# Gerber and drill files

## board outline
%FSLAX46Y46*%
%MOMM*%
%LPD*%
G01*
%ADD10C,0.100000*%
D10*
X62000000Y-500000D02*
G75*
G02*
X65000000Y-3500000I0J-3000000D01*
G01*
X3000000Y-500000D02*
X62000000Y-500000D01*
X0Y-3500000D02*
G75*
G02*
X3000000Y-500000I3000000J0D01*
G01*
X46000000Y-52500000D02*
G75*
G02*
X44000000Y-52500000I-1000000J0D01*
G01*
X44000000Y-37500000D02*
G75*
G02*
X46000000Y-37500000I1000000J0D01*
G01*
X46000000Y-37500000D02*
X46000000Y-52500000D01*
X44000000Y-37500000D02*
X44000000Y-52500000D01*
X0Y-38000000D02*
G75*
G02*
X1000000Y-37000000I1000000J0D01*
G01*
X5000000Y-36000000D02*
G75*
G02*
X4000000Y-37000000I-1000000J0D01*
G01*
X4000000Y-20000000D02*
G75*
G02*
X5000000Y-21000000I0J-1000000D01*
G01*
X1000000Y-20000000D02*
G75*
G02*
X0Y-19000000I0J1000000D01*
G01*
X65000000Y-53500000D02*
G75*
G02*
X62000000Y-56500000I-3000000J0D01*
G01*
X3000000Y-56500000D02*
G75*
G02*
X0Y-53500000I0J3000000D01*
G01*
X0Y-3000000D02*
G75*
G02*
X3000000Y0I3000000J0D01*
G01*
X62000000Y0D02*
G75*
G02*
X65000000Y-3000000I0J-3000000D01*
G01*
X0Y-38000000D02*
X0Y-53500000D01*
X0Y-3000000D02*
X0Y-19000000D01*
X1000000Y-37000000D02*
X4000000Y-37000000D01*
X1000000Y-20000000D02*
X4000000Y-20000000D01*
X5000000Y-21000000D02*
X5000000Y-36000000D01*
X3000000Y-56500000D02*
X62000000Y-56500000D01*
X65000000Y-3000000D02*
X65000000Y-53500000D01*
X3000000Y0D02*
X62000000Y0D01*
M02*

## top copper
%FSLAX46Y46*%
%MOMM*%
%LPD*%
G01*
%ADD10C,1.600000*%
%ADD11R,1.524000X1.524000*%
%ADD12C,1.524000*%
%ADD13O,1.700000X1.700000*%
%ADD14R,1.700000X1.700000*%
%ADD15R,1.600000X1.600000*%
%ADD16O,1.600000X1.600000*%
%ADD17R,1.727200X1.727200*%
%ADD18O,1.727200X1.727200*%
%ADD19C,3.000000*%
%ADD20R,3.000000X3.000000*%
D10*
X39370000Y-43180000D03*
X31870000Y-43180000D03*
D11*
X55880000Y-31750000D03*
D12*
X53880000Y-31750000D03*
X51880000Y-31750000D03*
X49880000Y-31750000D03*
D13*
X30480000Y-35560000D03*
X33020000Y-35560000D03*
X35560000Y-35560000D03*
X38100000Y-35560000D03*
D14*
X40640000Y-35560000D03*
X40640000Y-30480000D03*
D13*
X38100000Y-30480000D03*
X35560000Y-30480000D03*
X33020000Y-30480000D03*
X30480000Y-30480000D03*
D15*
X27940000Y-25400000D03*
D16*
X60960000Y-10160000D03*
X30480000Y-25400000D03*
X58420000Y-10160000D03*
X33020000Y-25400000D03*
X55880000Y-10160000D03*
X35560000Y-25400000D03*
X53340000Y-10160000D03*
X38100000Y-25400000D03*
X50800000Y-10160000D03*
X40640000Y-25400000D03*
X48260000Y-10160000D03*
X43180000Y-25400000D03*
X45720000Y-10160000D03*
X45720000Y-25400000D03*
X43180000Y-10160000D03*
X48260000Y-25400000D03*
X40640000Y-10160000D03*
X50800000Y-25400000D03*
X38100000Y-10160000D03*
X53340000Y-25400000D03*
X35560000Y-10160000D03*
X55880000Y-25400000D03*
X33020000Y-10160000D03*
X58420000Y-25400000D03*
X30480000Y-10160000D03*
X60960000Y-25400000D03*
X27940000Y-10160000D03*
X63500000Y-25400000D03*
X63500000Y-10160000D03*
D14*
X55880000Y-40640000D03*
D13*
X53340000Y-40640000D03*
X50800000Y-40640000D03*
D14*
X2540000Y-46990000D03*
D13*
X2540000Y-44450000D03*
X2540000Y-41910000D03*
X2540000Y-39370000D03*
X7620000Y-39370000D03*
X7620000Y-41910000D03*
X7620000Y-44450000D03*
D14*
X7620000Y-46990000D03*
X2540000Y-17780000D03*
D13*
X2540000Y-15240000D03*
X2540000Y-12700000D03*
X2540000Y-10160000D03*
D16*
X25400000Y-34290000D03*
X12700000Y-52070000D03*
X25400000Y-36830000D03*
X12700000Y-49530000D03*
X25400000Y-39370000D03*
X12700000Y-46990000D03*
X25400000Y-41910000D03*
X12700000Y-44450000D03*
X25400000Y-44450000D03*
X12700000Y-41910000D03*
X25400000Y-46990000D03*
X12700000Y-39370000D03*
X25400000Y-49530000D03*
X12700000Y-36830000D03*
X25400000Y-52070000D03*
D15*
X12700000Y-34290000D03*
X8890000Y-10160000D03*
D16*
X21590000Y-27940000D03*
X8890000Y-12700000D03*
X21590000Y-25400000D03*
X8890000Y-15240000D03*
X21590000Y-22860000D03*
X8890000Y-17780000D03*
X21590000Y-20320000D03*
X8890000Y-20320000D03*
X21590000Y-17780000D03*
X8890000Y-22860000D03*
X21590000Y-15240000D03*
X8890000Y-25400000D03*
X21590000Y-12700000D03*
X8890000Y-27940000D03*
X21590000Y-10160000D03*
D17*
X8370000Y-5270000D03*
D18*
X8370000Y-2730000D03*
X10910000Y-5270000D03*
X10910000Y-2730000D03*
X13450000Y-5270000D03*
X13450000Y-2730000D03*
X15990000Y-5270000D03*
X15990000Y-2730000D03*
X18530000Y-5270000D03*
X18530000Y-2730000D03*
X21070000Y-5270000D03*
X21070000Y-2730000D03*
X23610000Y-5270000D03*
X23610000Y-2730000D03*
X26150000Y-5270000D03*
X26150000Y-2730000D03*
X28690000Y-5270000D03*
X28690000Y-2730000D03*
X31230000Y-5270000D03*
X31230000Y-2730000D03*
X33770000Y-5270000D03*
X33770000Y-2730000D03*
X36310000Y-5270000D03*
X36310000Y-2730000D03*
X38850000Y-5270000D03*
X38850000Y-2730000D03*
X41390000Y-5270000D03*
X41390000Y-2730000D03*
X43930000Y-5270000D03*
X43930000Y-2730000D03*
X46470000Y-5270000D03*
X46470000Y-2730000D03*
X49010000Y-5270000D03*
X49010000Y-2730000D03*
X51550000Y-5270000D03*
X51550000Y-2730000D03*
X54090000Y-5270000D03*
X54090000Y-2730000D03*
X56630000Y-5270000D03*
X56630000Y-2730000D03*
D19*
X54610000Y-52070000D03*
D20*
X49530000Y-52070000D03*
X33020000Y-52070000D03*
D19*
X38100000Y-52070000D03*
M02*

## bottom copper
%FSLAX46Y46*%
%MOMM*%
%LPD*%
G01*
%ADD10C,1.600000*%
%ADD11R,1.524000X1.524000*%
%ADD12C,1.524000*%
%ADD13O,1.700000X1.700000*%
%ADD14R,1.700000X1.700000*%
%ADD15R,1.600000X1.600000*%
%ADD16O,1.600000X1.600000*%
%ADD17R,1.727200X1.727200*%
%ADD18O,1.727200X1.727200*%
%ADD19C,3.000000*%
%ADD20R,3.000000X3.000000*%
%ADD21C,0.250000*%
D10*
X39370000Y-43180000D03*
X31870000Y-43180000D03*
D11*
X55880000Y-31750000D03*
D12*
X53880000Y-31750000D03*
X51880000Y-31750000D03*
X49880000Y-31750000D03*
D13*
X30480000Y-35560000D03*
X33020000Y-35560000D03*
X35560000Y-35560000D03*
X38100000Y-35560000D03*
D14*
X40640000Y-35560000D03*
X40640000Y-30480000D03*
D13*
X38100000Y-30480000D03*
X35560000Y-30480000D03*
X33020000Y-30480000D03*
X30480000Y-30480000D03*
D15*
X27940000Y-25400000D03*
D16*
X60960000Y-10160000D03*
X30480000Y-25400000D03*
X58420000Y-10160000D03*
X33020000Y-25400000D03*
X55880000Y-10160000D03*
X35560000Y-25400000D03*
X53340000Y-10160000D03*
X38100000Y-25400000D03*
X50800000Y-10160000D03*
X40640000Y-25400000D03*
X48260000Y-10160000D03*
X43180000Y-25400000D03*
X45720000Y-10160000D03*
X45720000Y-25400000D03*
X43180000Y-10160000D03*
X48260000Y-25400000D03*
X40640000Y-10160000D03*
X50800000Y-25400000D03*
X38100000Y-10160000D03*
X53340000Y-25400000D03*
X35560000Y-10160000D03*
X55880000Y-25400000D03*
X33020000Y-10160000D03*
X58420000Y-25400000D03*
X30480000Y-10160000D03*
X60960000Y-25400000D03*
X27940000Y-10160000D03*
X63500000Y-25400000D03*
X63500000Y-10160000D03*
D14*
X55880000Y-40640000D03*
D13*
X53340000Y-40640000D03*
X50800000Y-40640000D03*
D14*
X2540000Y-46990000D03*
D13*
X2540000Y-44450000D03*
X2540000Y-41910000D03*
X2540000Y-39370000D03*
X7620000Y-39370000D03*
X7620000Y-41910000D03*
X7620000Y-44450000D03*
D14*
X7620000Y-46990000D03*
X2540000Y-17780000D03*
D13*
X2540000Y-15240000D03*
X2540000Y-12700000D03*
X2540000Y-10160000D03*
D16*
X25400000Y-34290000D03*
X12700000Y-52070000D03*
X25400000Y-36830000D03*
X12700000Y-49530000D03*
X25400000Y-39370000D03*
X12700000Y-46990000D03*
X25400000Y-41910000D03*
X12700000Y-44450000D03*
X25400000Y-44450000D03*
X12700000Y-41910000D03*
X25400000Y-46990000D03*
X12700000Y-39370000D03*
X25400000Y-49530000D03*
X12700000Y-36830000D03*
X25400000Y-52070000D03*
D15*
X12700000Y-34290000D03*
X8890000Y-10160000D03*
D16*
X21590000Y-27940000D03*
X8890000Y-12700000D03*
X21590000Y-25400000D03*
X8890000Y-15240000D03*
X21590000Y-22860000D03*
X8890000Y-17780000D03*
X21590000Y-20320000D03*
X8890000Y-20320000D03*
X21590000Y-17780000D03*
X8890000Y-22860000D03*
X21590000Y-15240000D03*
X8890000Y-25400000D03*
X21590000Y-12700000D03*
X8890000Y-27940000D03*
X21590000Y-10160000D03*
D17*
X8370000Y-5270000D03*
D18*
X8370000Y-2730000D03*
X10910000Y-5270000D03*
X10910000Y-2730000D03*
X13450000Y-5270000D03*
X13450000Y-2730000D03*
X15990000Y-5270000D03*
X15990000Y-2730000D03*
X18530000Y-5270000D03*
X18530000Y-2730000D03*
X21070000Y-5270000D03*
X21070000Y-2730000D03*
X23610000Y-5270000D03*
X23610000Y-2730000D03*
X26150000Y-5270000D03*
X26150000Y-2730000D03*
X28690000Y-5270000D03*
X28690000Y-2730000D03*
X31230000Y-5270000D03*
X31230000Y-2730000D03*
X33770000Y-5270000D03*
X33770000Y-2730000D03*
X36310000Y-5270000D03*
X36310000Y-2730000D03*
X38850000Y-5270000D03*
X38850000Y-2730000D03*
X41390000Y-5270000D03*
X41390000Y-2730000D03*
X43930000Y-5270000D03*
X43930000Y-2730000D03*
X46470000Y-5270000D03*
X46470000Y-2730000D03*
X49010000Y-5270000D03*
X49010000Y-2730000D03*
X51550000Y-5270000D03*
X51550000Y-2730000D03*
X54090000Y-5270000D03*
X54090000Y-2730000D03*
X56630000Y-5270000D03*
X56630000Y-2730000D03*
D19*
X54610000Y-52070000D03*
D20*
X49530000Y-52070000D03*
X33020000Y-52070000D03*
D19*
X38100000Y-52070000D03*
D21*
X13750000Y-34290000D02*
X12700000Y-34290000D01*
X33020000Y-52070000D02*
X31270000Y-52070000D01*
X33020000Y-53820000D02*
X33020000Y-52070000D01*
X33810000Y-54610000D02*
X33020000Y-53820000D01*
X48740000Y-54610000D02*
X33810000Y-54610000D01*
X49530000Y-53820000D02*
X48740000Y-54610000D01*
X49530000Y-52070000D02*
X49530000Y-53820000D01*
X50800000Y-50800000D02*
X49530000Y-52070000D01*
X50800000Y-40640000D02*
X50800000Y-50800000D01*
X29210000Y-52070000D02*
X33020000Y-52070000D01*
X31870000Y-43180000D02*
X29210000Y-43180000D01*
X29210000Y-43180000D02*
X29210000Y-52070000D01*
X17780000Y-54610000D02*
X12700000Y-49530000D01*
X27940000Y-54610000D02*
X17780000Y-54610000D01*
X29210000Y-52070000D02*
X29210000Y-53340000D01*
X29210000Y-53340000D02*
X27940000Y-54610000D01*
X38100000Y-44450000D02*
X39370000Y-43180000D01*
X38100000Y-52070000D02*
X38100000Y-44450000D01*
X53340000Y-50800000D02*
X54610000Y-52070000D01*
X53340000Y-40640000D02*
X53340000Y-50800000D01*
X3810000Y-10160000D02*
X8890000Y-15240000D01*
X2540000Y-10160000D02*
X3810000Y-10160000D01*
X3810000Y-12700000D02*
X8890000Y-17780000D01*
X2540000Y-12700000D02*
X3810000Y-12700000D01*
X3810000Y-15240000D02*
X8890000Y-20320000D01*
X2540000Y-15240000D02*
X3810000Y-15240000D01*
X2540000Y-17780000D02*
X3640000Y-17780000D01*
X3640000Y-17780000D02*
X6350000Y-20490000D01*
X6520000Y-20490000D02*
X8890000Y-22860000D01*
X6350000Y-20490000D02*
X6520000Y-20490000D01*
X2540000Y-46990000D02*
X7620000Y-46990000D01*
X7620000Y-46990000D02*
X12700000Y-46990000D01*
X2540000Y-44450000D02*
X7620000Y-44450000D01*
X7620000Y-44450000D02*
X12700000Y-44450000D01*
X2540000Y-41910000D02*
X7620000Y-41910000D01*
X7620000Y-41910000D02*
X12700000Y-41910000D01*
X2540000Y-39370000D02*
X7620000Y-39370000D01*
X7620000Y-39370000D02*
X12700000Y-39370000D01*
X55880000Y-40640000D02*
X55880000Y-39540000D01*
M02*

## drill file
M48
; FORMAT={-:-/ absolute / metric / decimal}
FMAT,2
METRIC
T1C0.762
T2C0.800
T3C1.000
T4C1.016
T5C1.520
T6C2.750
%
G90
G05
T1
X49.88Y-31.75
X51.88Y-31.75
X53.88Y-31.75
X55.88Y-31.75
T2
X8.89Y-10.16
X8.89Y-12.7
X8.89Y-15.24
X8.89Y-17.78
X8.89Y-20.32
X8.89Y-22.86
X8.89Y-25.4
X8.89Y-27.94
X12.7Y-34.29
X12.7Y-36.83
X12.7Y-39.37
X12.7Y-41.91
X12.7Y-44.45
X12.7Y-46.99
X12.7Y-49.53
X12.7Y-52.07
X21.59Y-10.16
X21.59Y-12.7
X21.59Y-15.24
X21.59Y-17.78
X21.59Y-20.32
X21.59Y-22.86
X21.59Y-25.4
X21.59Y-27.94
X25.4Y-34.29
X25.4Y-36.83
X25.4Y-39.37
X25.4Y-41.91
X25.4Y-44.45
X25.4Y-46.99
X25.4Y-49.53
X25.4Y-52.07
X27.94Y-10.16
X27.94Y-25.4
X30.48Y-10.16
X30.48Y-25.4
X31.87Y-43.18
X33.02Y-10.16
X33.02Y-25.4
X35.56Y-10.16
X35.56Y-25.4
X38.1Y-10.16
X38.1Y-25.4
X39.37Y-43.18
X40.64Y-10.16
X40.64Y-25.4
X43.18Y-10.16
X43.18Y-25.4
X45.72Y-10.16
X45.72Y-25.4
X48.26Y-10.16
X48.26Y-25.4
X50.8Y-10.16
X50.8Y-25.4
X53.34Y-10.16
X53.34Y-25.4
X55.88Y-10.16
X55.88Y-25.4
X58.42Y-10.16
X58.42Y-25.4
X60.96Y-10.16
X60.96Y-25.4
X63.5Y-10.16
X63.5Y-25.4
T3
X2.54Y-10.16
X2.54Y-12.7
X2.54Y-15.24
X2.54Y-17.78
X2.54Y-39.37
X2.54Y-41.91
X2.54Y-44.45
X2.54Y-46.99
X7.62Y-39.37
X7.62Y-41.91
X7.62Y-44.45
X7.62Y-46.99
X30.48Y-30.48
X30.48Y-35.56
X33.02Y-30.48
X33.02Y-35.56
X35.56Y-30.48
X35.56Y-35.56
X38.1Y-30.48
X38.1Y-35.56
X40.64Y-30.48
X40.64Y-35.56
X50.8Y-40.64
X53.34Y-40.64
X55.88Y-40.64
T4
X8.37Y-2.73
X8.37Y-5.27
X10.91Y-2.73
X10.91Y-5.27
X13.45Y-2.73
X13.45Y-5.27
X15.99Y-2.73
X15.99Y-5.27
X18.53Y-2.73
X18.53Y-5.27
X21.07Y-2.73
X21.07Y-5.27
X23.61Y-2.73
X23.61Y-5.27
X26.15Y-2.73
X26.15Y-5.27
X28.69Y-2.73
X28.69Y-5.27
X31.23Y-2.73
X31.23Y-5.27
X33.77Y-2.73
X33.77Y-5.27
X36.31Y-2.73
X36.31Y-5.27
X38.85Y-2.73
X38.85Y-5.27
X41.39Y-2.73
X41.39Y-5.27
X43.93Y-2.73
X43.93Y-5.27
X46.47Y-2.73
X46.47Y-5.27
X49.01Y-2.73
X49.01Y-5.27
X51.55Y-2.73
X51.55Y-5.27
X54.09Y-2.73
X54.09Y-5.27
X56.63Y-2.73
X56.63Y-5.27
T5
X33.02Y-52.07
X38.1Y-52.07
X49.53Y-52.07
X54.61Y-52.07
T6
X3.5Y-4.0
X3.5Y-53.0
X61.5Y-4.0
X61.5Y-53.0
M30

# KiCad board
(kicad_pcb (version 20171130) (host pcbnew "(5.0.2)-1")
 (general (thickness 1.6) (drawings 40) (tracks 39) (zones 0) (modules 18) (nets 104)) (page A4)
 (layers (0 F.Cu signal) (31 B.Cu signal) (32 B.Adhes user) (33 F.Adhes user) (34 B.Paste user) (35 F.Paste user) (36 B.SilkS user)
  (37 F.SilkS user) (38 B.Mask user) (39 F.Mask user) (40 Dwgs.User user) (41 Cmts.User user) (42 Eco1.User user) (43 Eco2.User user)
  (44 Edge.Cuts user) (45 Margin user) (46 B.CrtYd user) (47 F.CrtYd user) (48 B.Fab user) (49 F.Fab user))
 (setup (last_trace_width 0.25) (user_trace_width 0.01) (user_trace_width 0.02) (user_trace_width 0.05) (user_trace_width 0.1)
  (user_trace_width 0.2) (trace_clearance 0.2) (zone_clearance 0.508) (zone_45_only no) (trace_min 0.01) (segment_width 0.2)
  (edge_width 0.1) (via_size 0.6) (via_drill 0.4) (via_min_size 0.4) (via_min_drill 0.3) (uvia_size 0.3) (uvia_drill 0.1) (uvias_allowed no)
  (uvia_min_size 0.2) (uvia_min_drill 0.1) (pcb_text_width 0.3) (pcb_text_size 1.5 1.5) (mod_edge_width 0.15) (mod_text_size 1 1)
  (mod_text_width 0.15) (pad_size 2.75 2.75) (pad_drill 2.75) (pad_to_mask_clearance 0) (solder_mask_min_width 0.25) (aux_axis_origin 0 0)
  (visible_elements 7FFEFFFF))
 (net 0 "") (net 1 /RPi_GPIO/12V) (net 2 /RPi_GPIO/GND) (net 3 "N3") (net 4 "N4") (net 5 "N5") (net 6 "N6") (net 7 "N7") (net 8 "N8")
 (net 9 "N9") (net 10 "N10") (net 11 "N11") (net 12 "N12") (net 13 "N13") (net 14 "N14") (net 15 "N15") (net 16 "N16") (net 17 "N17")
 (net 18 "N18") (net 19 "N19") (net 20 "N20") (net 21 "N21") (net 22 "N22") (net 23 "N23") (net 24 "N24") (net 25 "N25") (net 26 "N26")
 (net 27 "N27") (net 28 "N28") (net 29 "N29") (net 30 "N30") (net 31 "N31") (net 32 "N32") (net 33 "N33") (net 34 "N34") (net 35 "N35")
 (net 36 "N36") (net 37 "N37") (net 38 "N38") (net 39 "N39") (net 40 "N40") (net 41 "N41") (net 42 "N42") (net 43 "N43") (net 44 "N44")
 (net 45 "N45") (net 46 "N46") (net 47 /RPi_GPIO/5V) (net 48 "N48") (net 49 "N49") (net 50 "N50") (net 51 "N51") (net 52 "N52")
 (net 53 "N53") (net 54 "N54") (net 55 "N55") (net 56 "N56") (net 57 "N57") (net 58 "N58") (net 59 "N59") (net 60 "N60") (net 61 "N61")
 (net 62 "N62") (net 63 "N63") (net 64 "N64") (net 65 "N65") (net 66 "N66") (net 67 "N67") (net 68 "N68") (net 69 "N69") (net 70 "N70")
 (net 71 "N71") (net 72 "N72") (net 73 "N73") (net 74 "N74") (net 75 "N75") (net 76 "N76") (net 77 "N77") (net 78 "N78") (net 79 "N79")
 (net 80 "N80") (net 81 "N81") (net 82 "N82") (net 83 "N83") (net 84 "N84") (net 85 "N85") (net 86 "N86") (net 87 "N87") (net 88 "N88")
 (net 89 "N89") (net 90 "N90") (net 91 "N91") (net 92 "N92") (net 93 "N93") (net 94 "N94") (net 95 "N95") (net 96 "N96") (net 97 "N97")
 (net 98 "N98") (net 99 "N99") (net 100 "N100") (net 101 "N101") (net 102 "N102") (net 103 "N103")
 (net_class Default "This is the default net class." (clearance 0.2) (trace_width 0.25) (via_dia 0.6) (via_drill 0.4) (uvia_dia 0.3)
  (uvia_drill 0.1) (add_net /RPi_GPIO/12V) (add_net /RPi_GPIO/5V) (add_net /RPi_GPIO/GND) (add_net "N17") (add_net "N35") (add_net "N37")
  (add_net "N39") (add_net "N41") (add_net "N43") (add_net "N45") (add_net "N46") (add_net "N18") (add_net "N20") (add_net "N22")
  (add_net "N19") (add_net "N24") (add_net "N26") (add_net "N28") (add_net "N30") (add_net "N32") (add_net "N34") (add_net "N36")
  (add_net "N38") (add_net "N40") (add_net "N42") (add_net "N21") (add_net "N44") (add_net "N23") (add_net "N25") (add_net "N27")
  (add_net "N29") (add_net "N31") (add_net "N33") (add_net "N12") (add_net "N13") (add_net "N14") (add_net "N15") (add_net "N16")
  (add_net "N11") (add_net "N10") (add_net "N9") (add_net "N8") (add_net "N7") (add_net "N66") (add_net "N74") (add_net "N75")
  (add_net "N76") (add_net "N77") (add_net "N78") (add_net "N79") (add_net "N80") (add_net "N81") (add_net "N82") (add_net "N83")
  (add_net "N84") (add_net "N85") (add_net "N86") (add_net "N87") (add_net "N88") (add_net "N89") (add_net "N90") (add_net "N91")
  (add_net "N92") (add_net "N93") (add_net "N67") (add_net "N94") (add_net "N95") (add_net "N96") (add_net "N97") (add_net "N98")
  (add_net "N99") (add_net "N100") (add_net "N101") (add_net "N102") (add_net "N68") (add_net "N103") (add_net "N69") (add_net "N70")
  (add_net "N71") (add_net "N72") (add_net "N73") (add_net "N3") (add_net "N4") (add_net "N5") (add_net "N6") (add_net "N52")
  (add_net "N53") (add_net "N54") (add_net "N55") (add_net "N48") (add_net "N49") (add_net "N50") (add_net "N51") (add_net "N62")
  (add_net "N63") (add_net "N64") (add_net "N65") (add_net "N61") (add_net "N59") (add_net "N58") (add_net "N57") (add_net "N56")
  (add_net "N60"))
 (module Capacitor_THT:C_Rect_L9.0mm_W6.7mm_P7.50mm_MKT (layer F.Cu) (at 39.37 43.18 180)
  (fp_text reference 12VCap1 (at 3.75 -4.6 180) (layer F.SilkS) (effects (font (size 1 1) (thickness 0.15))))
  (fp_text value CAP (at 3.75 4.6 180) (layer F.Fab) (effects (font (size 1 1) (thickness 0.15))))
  (pad 1 thru_hole circle (at 0 0 180) (size 1.6 1.6) (drill 0.8) (layers *.Cu *.Mask) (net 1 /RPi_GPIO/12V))
  (pad 2 thru_hole circle (at 7.5 0 180) (size 1.6 1.6) (drill 0.8) (layers *.Cu *.Mask) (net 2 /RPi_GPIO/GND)))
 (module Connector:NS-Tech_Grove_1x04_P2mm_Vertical (layer F.Cu) (at 55.88 31.75 270)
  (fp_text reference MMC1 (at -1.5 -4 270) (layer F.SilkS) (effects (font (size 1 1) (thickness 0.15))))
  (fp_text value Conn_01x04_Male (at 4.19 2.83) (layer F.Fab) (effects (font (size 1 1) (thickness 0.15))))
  (pad 1 thru_hole rect (at 0 0 270) (size 1.524 1.524) (drill 0.762) (layers *.Cu *.Mask) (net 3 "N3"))
  (pad 2 thru_hole circle (at 0 2 270) (size 1.524 1.524) (drill 0.762) (layers *.Cu *.Mask) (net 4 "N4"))
  (pad 3 thru_hole circle (at 0 4 270) (size 1.524 1.524) (drill 0.762) (layers *.Cu *.Mask) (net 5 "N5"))
  (pad 4 thru_hole circle (at 0 6 270) (size 1.524 1.524) (drill 0.762) (layers *.Cu *.Mask) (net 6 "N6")))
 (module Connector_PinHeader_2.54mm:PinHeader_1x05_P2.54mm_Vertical (layer F.Cu) (at 40.64 35.56 270)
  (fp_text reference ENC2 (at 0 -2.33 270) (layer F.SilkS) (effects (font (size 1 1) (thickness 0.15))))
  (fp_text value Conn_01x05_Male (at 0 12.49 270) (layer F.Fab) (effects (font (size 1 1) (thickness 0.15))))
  (pad 5 thru_hole oval (at 0 10.16 270) (size 1.7 1.7) (drill 1) (layers *.Cu *.Mask) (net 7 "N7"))
  (pad 4 thru_hole oval (at 0 7.62 270) (size 1.7 1.7) (drill 1) (layers *.Cu *.Mask) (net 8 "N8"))
  (pad 3 thru_hole oval (at 0 5.08 270) (size 1.7 1.7) (drill 1) (layers *.Cu *.Mask) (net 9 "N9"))
  (pad 2 thru_hole oval (at 0 2.54 270) (size 1.7 1.7) (drill 1) (layers *.Cu *.Mask) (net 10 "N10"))
  (pad 1 thru_hole rect (at 0 0 270) (size 1.7 1.7) (drill 1) (layers *.Cu *.Mask) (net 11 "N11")))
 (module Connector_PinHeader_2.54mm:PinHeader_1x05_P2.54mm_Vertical (layer F.Cu) (at 40.64 30.48 270)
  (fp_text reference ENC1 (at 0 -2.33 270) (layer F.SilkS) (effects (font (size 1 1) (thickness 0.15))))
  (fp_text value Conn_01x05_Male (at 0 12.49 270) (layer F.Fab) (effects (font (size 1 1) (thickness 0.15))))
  (pad 1 thru_hole rect (at 0 0 270) (size 1.7 1.7) (drill 1) (layers *.Cu *.Mask) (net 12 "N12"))
  (pad 2 thru_hole oval (at 0 2.54 270) (size 1.7 1.7) (drill 1) (layers *.Cu *.Mask) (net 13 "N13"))
  (pad 3 thru_hole oval (at 0 5.08 270) (size 1.7 1.7) (drill 1) (layers *.Cu *.Mask) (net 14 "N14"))
  (pad 4 thru_hole oval (at 0 7.62 270) (size 1.7 1.7) (drill 1) (layers *.Cu *.Mask) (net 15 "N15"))
  (pad 5 thru_hole oval (at 0 10.16 270) (size 1.7 1.7) (drill 1) (layers *.Cu *.Mask) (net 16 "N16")))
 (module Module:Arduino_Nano (layer F.Cu) (at 27.94 25.4 90)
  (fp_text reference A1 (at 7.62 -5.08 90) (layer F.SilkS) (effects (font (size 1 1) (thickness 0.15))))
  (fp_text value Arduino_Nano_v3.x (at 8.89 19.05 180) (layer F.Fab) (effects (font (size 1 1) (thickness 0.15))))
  (pad 1 thru_hole rect (at 0 0 90) (size 1.6 1.6) (drill 0.8) (layers *.Cu *.Mask) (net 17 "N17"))
  (pad 17 thru_hole oval (at 15.24 33.02 90) (size 1.6 1.6) (drill 0.8) (layers *.Cu *.Mask) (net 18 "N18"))
  (pad 2 thru_hole oval (at 0 2.54 90) (size 1.6 1.6) (drill 0.8) (layers *.Cu *.Mask) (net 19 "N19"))
  (pad 18 thru_hole oval (at 15.24 30.48 90) (size 1.6 1.6) (drill 0.8) (layers *.Cu *.Mask) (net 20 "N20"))
  (pad 3 thru_hole oval (at 0 5.08 90) (size 1.6 1.6) (drill 0.8) (layers *.Cu *.Mask) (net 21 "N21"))
  (pad 19 thru_hole oval (at 15.24 27.94 90) (size 1.6 1.6) (drill 0.8) (layers *.Cu *.Mask) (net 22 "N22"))
  (pad 4 thru_hole oval (at 0 7.62 90) (size 1.6 1.6) (drill 0.8) (layers *.Cu *.Mask) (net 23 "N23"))
  (pad 20 thru_hole oval (at 15.24 25.4 90) (size 1.6 1.6) (drill 0.8) (layers *.Cu *.Mask) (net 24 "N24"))
  (pad 5 thru_hole oval (at 0 10.16 90) (size 1.6 1.6) (drill 0.8) (layers *.Cu *.Mask) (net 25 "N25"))
  (pad 21 thru_hole oval (at 15.24 22.86 90) (size 1.6 1.6) (drill 0.8) (layers *.Cu *.Mask) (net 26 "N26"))
  (pad 6 thru_hole oval (at 0 12.7 90) (size 1.6 1.6) (drill 0.8) (layers *.Cu *.Mask) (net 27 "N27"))
  (pad 22 thru_hole oval (at 15.24 20.32 90) (size 1.6 1.6) (drill 0.8) (layers *.Cu *.Mask) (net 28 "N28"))
  (pad 7 thru_hole oval (at 0 15.24 90) (size 1.6 1.6) (drill 0.8) (layers *.Cu *.Mask) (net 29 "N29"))
  (pad 23 thru_hole oval (at 15.24 17.78 90) (size 1.6 1.6) (drill 0.8) (layers *.Cu *.Mask) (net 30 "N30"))
  (pad 8 thru_hole oval (at 0 17.78 90) (size 1.6 1.6) (drill 0.8) (layers *.Cu *.Mask) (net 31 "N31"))
  (pad 24 thru_hole oval (at 15.24 15.24 90) (size 1.6 1.6) (drill 0.8) (layers *.Cu *.Mask) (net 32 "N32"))
  (pad 9 thru_hole oval (at 0 20.32 90) (size 1.6 1.6) (drill 0.8) (layers *.Cu *.Mask) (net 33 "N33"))
  (pad 25 thru_hole oval (at 15.24 12.7 90) (size 1.6 1.6) (drill 0.8) (layers *.Cu *.Mask) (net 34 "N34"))
  (pad 10 thru_hole oval (at 0 22.86 90) (size 1.6 1.6) (drill 0.8) (layers *.Cu *.Mask) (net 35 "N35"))
  (pad 26 thru_hole oval (at 15.24 10.16 90) (size 1.6 1.6) (drill 0.8) (layers *.Cu *.Mask) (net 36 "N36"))
  (pad 11 thru_hole oval (at 0 25.4 90) (size 1.6 1.6) (drill 0.8) (layers *.Cu *.Mask) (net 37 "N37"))
  (pad 27 thru_hole oval (at 15.24 7.62 90) (size 1.6 1.6) (drill 0.8) (layers *.Cu *.Mask) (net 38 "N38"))
  (pad 12 thru_hole oval (at 0 27.94 90) (size 1.6 1.6) (drill 0.8) (layers *.Cu *.Mask) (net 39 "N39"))
  (pad 28 thru_hole oval (at 15.24 5.08 90) (size 1.6 1.6) (drill 0.8) (layers *.Cu *.Mask) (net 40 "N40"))
  (pad 13 thru_hole oval (at 0 30.48 90) (size 1.6 1.6) (drill 0.8) (layers *.Cu *.Mask) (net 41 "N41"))
  (pad 29 thru_hole oval (at 15.24 2.54 90) (size 1.6 1.6) (drill 0.8) (layers *.Cu *.Mask) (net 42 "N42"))
  (pad 14 thru_hole oval (at 0 33.02 90) (size 1.6 1.6) (drill 0.8) (layers *.Cu *.Mask) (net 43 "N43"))
  (pad 30 thru_hole oval (at 15.24 0 90) (size 1.6 1.6) (drill 0.8) (layers *.Cu *.Mask) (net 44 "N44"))
  (pad 15 thru_hole oval (at 0 35.56 90) (size 1.6 1.6) (drill 0.8) (layers *.Cu *.Mask) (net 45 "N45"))
  (pad 16 thru_hole oval (at 15.24 35.56 90) (size 1.6 1.6) (drill 0.8) (layers *.Cu *.Mask) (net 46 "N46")))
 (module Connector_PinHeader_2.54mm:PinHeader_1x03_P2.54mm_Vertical (layer F.Cu) (at 55.88 40.64 270)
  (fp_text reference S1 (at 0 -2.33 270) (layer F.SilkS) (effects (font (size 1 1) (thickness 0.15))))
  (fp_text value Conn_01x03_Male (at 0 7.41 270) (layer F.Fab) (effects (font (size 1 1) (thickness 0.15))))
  (pad 1 thru_hole rect (at 0 0 270) (size 1.7 1.7) (drill 1) (layers *.Cu *.Mask) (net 27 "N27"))
  (pad 2 thru_hole oval (at 0 2.54 270) (size 1.7 1.7) (drill 1) (layers *.Cu *.Mask) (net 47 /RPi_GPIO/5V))
  (pad 3 thru_hole oval (at 0 5.08 270) (size 1.7 1.7) (drill 1) (layers *.Cu *.Mask) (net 2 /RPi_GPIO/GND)))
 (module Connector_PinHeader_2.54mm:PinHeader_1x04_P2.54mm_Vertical (layer F.Cu) (at 2.54 46.99 180)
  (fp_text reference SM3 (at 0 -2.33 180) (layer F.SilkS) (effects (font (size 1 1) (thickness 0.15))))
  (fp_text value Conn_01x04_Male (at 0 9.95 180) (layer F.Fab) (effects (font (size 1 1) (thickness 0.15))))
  (pad 1 thru_hole rect (at 0 0 180) (size 1.7 1.7) (drill 1) (layers *.Cu *.Mask) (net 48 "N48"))
  (pad 2 thru_hole oval (at 0 2.54 180) (size 1.7 1.7) (drill 1) (layers *.Cu *.Mask) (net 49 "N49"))
  (pad 3 thru_hole oval (at 0 5.08 180) (size 1.7 1.7) (drill 1) (layers *.Cu *.Mask) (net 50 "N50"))
  (pad 4 thru_hole oval (at 0 7.62 180) (size 1.7 1.7) (drill 1) (layers *.Cu *.Mask) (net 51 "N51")))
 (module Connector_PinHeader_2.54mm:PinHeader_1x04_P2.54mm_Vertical (layer F.Cu) (at 7.62 46.99 180)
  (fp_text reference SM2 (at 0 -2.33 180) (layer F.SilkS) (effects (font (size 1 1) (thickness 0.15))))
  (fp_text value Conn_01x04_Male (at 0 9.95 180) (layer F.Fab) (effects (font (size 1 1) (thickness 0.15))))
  (pad 4 thru_hole oval (at 0 7.62 180) (size 1.7 1.7) (drill 1) (layers *.Cu *.Mask) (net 51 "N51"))
  (pad 3 thru_hole oval (at 0 5.08 180) (size 1.7 1.7) (drill 1) (layers *.Cu *.Mask) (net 50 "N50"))
  (pad 2 thru_hole oval (at 0 2.54 180) (size 1.7 1.7) (drill 1) (layers *.Cu *.Mask) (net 49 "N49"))
  (pad 1 thru_hole rect (at 0 0 180) (size 1.7 1.7) (drill 1) (layers *.Cu *.Mask) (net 48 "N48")))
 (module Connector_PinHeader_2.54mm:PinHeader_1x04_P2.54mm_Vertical (layer F.Cu) (at 2.54 17.78 180)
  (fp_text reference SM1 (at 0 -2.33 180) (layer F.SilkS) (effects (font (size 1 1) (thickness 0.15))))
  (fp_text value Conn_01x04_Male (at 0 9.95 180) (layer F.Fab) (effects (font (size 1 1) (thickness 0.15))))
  (pad 1 thru_hole rect (at 0 0 180) (size 1.7 1.7) (drill 1) (layers *.Cu *.Mask) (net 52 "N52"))
  (pad 2 thru_hole oval (at 0 2.54 180) (size 1.7 1.7) (drill 1) (layers *.Cu *.Mask) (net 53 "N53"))
  (pad 3 thru_hole oval (at 0 5.08 180) (size 1.7 1.7) (drill 1) (layers *.Cu *.Mask) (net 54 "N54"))
  (pad 4 thru_hole oval (at 0 7.62 180) (size 1.7 1.7) (drill 1) (layers *.Cu *.Mask) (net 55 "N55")))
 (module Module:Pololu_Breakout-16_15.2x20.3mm (layer F.Cu) (at 12.7 34.29)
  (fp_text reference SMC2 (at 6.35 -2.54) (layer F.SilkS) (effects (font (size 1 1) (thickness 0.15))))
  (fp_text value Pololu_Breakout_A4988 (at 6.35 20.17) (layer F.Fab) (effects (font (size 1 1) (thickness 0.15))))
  (pad 16 thru_hole oval (at 12.7 0) (size 1.6 1.6) (drill 0.8) (layers *.Cu *.Mask) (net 45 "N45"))
  (pad 8 thru_hole oval (at 0 17.78) (size 1.6 1.6) (drill 0.8) (layers *.Cu *.Mask) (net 1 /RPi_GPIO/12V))
  (pad 15 thru_hole oval (at 12.7 2.54) (size 1.6 1.6) (drill 0.8) (layers *.Cu *.Mask) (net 43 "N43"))
  (pad 7 thru_hole oval (at 0 15.24) (size 1.6 1.6) (drill 0.8) (layers *.Cu *.Mask) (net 2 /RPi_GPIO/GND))
  (pad 14 thru_hole oval (at 12.7 5.08) (size 1.6 1.6) (drill 0.8) (layers *.Cu *.Mask) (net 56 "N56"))
  (pad 6 thru_hole oval (at 0 12.7) (size 1.6 1.6) (drill 0.8) (layers *.Cu *.Mask) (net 48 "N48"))
  (pad 13 thru_hole oval (at 12.7 7.62) (size 1.6 1.6) (drill 0.8) (layers *.Cu *.Mask) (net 56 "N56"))
  (pad 5 thru_hole oval (at 0 10.16) (size 1.6 1.6) (drill 0.8) (layers *.Cu *.Mask) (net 49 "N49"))
  (pad 12 thru_hole oval (at 12.7 10.16) (size 1.6 1.6) (drill 0.8) (layers *.Cu *.Mask) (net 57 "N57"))
  (pad 4 thru_hole oval (at 0 7.62) (size 1.6 1.6) (drill 0.8) (layers *.Cu *.Mask) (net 50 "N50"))
  (pad 11 thru_hole oval (at 12.7 12.7) (size 1.6 1.6) (drill 0.8) (layers *.Cu *.Mask) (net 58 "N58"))
  (pad 3 thru_hole oval (at 0 5.08) (size 1.6 1.6) (drill 0.8) (layers *.Cu *.Mask) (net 51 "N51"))
  (pad 10 thru_hole oval (at 12.7 15.24) (size 1.6 1.6) (drill 0.8) (layers *.Cu *.Mask) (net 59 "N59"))
  (pad 2 thru_hole oval (at 0 2.54) (size 1.6 1.6) (drill 0.8) (layers *.Cu *.Mask) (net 47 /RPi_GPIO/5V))
  (pad 9 thru_hole oval (at 12.7 17.78) (size 1.6 1.6) (drill 0.8) (layers *.Cu *.Mask) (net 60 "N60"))
  (pad 1 thru_hole rect (at 0 0) (size 1.6 1.6) (drill 0.8) (layers *.Cu *.Mask) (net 2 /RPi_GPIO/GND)))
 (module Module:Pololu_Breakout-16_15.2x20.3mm (layer F.Cu) (at 8.89 10.16)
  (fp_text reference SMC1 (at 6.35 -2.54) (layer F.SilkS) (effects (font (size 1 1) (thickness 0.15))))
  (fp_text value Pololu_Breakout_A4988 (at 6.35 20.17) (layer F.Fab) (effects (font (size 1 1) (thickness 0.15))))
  (pad 1 thru_hole rect (at 0 0) (size 1.6 1.6) (drill 0.8) (layers *.Cu *.Mask) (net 2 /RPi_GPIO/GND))
  (pad 9 thru_hole oval (at 12.7 17.78) (size 1.6 1.6) (drill 0.8) (layers *.Cu *.Mask) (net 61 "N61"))
  (pad 2 thru_hole oval (at 0 2.54) (size 1.6 1.6) (drill 0.8) (layers *.Cu *.Mask) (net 47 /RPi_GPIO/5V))
  (pad 10 thru_hole oval (at 12.7 15.24) (size 1.6 1.6) (drill 0.8) (layers *.Cu *.Mask) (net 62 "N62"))
  (pad 3 thru_hole oval (at 0 5.08) (size 1.6 1.6) (drill 0.8) (layers *.Cu *.Mask) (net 55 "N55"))
  (pad 11 thru_hole oval (at 12.7 12.7) (size 1.6 1.6) (drill 0.8) (layers *.Cu *.Mask) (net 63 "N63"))
  (pad 4 thru_hole oval (at 0 7.62) (size 1.6 1.6) (drill 0.8) (layers *.Cu *.Mask) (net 54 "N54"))
  (pad 12 thru_hole oval (at 12.7 10.16) (size 1.6 1.6) (drill 0.8) (layers *.Cu *.Mask) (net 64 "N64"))
  (pad 5 thru_hole oval (at 0 10.16) (size 1.6 1.6) (drill 0.8) (layers *.Cu *.Mask) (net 53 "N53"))
  (pad 13 thru_hole oval (at 12.7 7.62) (size 1.6 1.6) (drill 0.8) (layers *.Cu *.Mask) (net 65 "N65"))
  (pad 6 thru_hole oval (at 0 12.7) (size 1.6 1.6) (drill 0.8) (layers *.Cu *.Mask) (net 52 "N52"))
  (pad 14 thru_hole oval (at 12.7 5.08) (size 1.6 1.6) (drill 0.8) (layers *.Cu *.Mask) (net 65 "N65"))
  (pad 7 thru_hole oval (at 0 15.24) (size 1.6 1.6) (drill 0.8) (layers *.Cu *.Mask) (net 2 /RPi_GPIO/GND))
  (pad 15 thru_hole oval (at 12.7 2.54) (size 1.6 1.6) (drill 0.8) (layers *.Cu *.Mask) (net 39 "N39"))
  (pad 8 thru_hole oval (at 0 17.78) (size 1.6 1.6) (drill 0.8) (layers *.Cu *.Mask) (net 1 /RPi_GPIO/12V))
  (pad 16 thru_hole oval (at 12.7 0) (size 1.6 1.6) (drill 0.8) (layers *.Cu *.Mask) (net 37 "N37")))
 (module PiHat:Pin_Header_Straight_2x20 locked (layer F.Cu) (at 32.5 4 90)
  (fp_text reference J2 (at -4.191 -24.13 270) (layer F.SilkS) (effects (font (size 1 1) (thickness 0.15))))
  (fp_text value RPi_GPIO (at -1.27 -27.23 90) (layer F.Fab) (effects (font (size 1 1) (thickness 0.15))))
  (pad 1 thru_hole rect (at -1.27 -24.13 90) (size 1.7272 1.7272) (drill 1.016) (layers *.Cu *.Mask F.SilkS) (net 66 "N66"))
  (pad 2 thru_hole oval (at 1.27 -24.13 90) (size 1.7272 1.7272) (drill 1.016) (layers *.Cu *.Mask F.SilkS) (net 47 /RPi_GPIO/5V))
  (pad 3 thru_hole oval (at -1.27 -21.59 90) (size 1.7272 1.7272) (drill 1.016) (layers *.Cu *.Mask F.SilkS) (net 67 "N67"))
  (pad 4 thru_hole oval (at 1.27 -21.59 90) (size 1.7272 1.7272) (drill 1.016) (layers *.Cu *.Mask F.SilkS) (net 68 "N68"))
  (pad 5 thru_hole oval (at -1.27 -19.05 90) (size 1.7272 1.7272) (drill 1.016) (layers *.Cu *.Mask F.SilkS) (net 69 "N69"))
  (pad 6 thru_hole oval (at 1.27 -19.05 90) (size 1.7272 1.7272) (drill 1.016) (layers *.Cu *.Mask F.SilkS) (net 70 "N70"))
  (pad 7 thru_hole oval (at -1.27 -16.51 90) (size 1.7272 1.7272) (drill 1.016) (layers *.Cu *.Mask F.SilkS) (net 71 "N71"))
  (pad 8 thru_hole oval (at 1.27 -16.51 90) (size 1.7272 1.7272) (drill 1.016) (layers *.Cu *.Mask F.SilkS) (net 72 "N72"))
  (pad 9 thru_hole oval (at -1.27 -13.97 90) (size 1.7272 1.7272) (drill 1.016) (layers *.Cu *.Mask F.SilkS) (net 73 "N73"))
  (pad 10 thru_hole oval (at 1.27 -13.97 90) (size 1.7272 1.7272) (drill 1.016) (layers *.Cu *.Mask F.SilkS) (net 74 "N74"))
  (pad 11 thru_hole oval (at -1.27 -11.43 90) (size 1.7272 1.7272) (drill 1.016) (layers *.Cu *.Mask F.SilkS) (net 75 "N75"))
  (pad 12 thru_hole oval (at 1.27 -11.43 90) (size 1.7272 1.7272) (drill 1.016) (layers *.Cu *.Mask F.SilkS) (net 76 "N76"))
  (pad 13 thru_hole oval (at -1.27 -8.89 90) (size 1.7272 1.7272) (drill 1.016) (layers *.Cu *.Mask F.SilkS) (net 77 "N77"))
  (pad 14 thru_hole oval (at 1.27 -8.89 90) (size 1.7272 1.7272) (drill 1.016) (layers *.Cu *.Mask F.SilkS) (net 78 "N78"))
  (pad 15 thru_hole oval (at -1.27 -6.35 90) (size 1.7272 1.7272) (drill 1.016) (layers *.Cu *.Mask F.SilkS) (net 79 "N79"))
  (pad 16 thru_hole oval (at 1.27 -6.35 90) (size 1.7272 1.7272) (drill 1.016) (layers *.Cu *.Mask F.SilkS) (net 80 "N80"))
  (pad 17 thru_hole oval (at -1.27 -3.81 90) (size 1.7272 1.7272) (drill 1.016) (layers *.Cu *.Mask F.SilkS) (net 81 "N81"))
  (pad 18 thru_hole oval (at 1.27 -3.81 90) (size 1.7272 1.7272) (drill 1.016) (layers *.Cu *.Mask F.SilkS) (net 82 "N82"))
  (pad 19 thru_hole oval (at -1.27 -1.27 90) (size 1.7272 1.7272) (drill 1.016) (layers *.Cu *.Mask F.SilkS) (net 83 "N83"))
  (pad 20 thru_hole oval (at 1.27 -1.27 90) (size 1.7272 1.7272) (drill 1.016) (layers *.Cu *.Mask F.SilkS) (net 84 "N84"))
  (pad 21 thru_hole oval (at -1.27 1.27 90) (size 1.7272 1.7272) (drill 1.016) (layers *.Cu *.Mask F.SilkS) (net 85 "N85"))
  (pad 22 thru_hole oval (at 1.27 1.27 90) (size 1.7272 1.7272) (drill 1.016) (layers *.Cu *.Mask F.SilkS) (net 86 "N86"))
  (pad 23 thru_hole oval (at -1.27 3.81 90) (size 1.7272 1.7272) (drill 1.016) (layers *.Cu *.Mask F.SilkS) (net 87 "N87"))
  (pad 24 thru_hole oval (at 1.27 3.81 90) (size 1.7272 1.7272) (drill 1.016) (layers *.Cu *.Mask F.SilkS) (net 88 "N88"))
  (pad 25 thru_hole oval (at -1.27 6.35 90) (size 1.7272 1.7272) (drill 1.016) (layers *.Cu *.Mask F.SilkS) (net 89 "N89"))
  (pad 26 thru_hole oval (at 1.27 6.35 90) (size 1.7272 1.7272) (drill 1.016) (layers *.Cu *.Mask F.SilkS) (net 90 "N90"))
  (pad 27 thru_hole oval (at -1.27 8.89 90) (size 1.7272 1.7272) (drill 1.016) (layers *.Cu *.Mask F.SilkS) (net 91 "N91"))
  (pad 28 thru_hole oval (at 1.27 8.89 90) (size 1.7272 1.7272) (drill 1.016) (layers *.Cu *.Mask F.SilkS) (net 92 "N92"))
  (pad 29 thru_hole oval (at -1.27 11.43 90) (size 1.7272 1.7272) (drill 1.016) (layers *.Cu *.Mask F.SilkS) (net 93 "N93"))
  (pad 30 thru_hole oval (at 1.27 11.43 90) (size 1.7272 1.7272) (drill 1.016) (layers *.Cu *.Mask F.SilkS) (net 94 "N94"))
  (pad 31 thru_hole oval (at -1.27 13.97 90) (size 1.7272 1.7272) (drill 1.016) (layers *.Cu *.Mask F.SilkS) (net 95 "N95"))
  (pad 32 thru_hole oval (at 1.27 13.97 90) (size 1.7272 1.7272) (drill 1.016) (layers *.Cu *.Mask F.SilkS) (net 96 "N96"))
  (pad 33 thru_hole oval (at -1.27 16.51 90) (size 1.7272 1.7272) (drill 1.016) (layers *.Cu *.Mask F.SilkS) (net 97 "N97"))
  (pad 34 thru_hole oval (at 1.27 16.51 90) (size 1.7272 1.7272) (drill 1.016) (layers *.Cu *.Mask F.SilkS) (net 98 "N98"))
  (pad 35 thru_hole oval (at -1.27 19.05 90) (size 1.7272 1.7272) (drill 1.016) (layers *.Cu *.Mask F.SilkS) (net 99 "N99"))
  (pad 36 thru_hole oval (at 1.27 19.05 90) (size 1.7272 1.7272) (drill 1.016) (layers *.Cu *.Mask F.SilkS) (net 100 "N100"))
  (pad 37 thru_hole oval (at -1.27 21.59 90) (size 1.7272 1.7272) (drill 1.016) (layers *.Cu *.Mask F.SilkS) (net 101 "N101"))
  (pad 38 thru_hole oval (at 1.27 21.59 90) (size 1.7272 1.7272) (drill 1.016) (layers *.Cu *.Mask F.SilkS) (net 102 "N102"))
  (pad 39 thru_hole oval (at -1.27 24.13 90) (size 1.7272 1.7272) (drill 1.016) (layers *.Cu *.Mask F.SilkS) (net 2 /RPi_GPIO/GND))
  (pad 40 thru_hole oval (at 1.27 24.13 90) (size 1.7272 1.7272) (drill 1.016) (layers *.Cu *.Mask F.SilkS) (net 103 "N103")))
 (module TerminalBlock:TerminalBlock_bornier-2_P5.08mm (layer F.Cu) (at 49.53 52.07)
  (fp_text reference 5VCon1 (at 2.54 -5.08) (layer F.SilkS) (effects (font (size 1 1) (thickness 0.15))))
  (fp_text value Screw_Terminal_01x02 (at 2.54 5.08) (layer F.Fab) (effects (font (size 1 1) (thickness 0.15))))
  (pad 2 thru_hole circle (at 5.08 0) (size 3 3) (drill 1.52) (layers *.Cu *.Mask) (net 47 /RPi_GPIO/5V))
  (pad 1 thru_hole rect (at 0 0) (size 3 3) (drill 1.52) (layers *.Cu *.Mask) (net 2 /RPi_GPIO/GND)))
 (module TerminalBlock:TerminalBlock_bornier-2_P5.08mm (layer F.Cu) (at 33.02 52.07)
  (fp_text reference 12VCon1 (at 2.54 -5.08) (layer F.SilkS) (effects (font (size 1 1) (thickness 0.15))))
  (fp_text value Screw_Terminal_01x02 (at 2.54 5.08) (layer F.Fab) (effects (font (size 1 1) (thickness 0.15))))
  (pad 1 thru_hole rect (at 0 0) (size 3 3) (drill 1.52) (layers *.Cu *.Mask) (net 2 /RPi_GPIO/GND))
  (pad 2 thru_hole circle (at 5.08 0) (size 3 3) (drill 1.52) (layers *.Cu *.Mask) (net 1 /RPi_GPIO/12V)))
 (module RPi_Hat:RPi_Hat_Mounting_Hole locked (layer F.Cu) (at 61.5 4)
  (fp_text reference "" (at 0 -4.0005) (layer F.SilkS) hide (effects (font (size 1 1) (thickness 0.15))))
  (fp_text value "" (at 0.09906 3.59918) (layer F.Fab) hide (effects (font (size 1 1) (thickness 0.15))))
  (pad "" np_thru_hole circle (at 0 0) (size 2.75 2.75) (drill 2.75) (layers *.Cu *.Mask) (solder_mask_margin 1.725) (clearance 1.725)))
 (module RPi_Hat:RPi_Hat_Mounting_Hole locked (layer F.Cu) (at 61.5 53)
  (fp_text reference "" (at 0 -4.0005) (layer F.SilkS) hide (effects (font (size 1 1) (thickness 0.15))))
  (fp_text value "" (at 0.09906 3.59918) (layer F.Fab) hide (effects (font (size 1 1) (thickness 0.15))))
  (pad "" np_thru_hole circle (at 0 0) (size 2.75 2.75) (drill 2.75) (layers *.Cu *.Mask) (solder_mask_margin 1.725) (clearance 1.725)))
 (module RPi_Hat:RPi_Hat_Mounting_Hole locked (layer F.Cu) (at 3.5 53)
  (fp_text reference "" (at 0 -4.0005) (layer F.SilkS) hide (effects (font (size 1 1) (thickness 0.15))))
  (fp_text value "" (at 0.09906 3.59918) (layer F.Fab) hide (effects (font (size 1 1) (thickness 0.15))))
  (pad "" np_thru_hole circle (at 0 0) (size 2.75 2.75) (drill 2.75) (layers *.Cu *.Mask) (solder_mask_margin 1.725) (clearance 1.725)))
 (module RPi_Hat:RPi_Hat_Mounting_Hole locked (layer F.Cu) (at 3.5 4)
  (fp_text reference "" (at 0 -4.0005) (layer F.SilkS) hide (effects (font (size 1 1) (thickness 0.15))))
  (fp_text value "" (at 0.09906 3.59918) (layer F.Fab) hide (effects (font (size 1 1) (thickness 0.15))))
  (pad "" np_thru_hole circle (at 0 0) (size 2.75 2.75) (drill 2.75) (layers *.Cu *.Mask) (solder_mask_margin 1.725) (clearance 1.725)))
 (gr_arc (start 62 3.5) (end 62 0.5) (angle 90) (layer Edge.Cuts) (width 0.1))
 (gr_line (start 3 0.5) (end 62 0.5) (angle 90) (layer Edge.Cuts) (width 0.1))
 (gr_arc (start 3 3.5) (end 0 3.5) (angle 90) (layer Edge.Cuts) (width 0.1))
 (gr_arc (start 45 52.5) (end 44 52.5) (angle -180) (layer Edge.Cuts) (width 0.1))
 (gr_arc (start 45 37.5) (end 44 37.5) (angle 180) (layer Edge.Cuts) (width 0.1))
 (gr_line (start 46 37.5) (end 46 52.5) (angle 90) (layer Edge.Cuts) (width 0.1))
 (gr_line (start 44 37.5) (end 44 52.5) (angle 90) (layer Edge.Cuts) (width 0.1))
 (gr_arc (start 1 38) (end 0 38) (angle 90) (layer Edge.Cuts) (width 0.1))
 (gr_arc (start 4 36) (end 5 36) (angle 90) (layer Edge.Cuts) (width 0.1))
 (gr_arc (start 4 21) (end 4 20) (angle 90) (layer Edge.Cuts) (width 0.1))
 (gr_arc (start 1 19) (end 1 20) (angle 90) (layer Edge.Cuts) (width 0.1))
 (gr_arc (start 62 53.5) (end 65 53.5) (angle 90) (layer Edge.Cuts) (width 0.1))
 (gr_arc (start 3 53.5) (end 3 56.5) (angle 90) (layer Edge.Cuts) (width 0.1))
 (gr_arc (start 3 3) (end 0 3) (angle 90) (layer Edge.Cuts) (width 0.1))
 (gr_arc (start 62 3) (end 62 0) (angle 90) (layer Edge.Cuts) (width 0.1))
 (gr_line (start 0 38) (end 0 53.5) (layer Edge.Cuts) (width 0.1))
 (gr_line (start 0 3) (end 0 19) (layer Edge.Cuts) (width 0.1))
 (gr_line (start 1 37) (end 4 37) (layer Edge.Cuts) (width 0.1))
 (gr_line (start 1 20) (end 4 20) (layer Edge.Cuts) (width 0.1))
 (gr_line (start 5 21) (end 5 36) (layer Edge.Cuts) (width 0.1))
 (gr_line (start 3 56.5) (end 62 56.5) (angle 90) (layer Edge.Cuts) (width 0.1))
 (gr_line (start 65 3) (end 65 53.5) (angle 90) (layer Edge.Cuts) (width 0.1))
 (gr_line (start 3 0) (end 62 0) (angle 90) (layer Edge.Cuts) (width 0.1))
 (segment (start 13.75 34.29) (end 12.7 34.29) (width 0.25) (layer B.Cu) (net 2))
 (segment (start 33.02 52.07) (end 31.27 52.07) (width 0.25) (layer B.Cu) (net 2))
 (segment (start 33.02 53.82) (end 33.02 52.07) (width 0.25) (layer B.Cu) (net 2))
 (segment (start 33.81 54.61) (end 33.02 53.82) (width 0.25) (layer B.Cu) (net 2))
 (segment (start 48.74 54.61) (end 33.81 54.61) (width 0.25) (layer B.Cu) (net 2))
 (segment (start 49.53 53.82) (end 48.74 54.61) (width 0.25) (layer B.Cu) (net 2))
 (segment (start 49.53 52.07) (end 49.53 53.82) (width 0.25) (layer B.Cu) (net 2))
 (segment (start 50.8 50.8) (end 49.53 52.07) (width 0.25) (layer B.Cu) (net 2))
 (segment (start 50.8 40.64) (end 50.8 50.8) (width 0.25) (layer B.Cu) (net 2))
 (segment (start 29.21 52.07) (end 33.02 52.07) (width 0.25) (layer B.Cu) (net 2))
 (segment (start 31.87 43.18) (end 29.21 43.18) (width 0.25) (layer B.Cu) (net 2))
 (segment (start 29.21 43.18) (end 29.21 52.07) (width 0.25) (layer B.Cu) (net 2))
 (segment (start 17.78 54.61) (end 12.7 49.53) (width 0.25) (layer B.Cu) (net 2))
 (segment (start 27.94 54.61) (end 17.78 54.61) (width 0.25) (layer B.Cu) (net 2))
 (segment (start 29.21 52.07) (end 29.21 53.34) (width 0.25) (layer B.Cu) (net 2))
 (segment (start 29.21 53.34) (end 27.94 54.61) (width 0.25) (layer B.Cu) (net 2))
 (segment (start 38.1 44.45) (end 39.37 43.18) (width 0.25) (layer B.Cu) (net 1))
 (segment (start 38.1 52.07) (end 38.1 44.45) (width 0.25) (layer B.Cu) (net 1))
 (segment (start 53.34 50.8) (end 54.61 52.07) (width 0.25) (layer B.Cu) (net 47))
 (segment (start 53.34 40.64) (end 53.34 50.8) (width 0.25) (layer B.Cu) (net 47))
 (segment (start 3.81 10.16) (end 8.89 15.24) (width 0.25) (layer B.Cu) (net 55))
 (segment (start 2.54 10.16) (end 3.81 10.16) (width 0.25) (layer B.Cu) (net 55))
 (segment (start 3.81 12.7) (end 8.89 17.78) (width 0.25) (layer B.Cu) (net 54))
 (segment (start 2.54 12.7) (end 3.81 12.7) (width 0.25) (layer B.Cu) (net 54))
 (segment (start 3.81 15.24) (end 8.89 20.32) (width 0.25) (layer B.Cu) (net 53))
 (segment (start 2.54 15.24) (end 3.81 15.24) (width 0.25) (layer B.Cu) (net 53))
 (segment (start 2.54 17.78) (end 3.64 17.78) (width 0.25) (layer B.Cu) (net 52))
 (segment (start 3.64 17.78) (end 6.35 20.49) (width 0.25) (layer B.Cu) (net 52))
 (segment (start 6.52 20.49) (end 8.89 22.86) (width 0.25) (layer B.Cu) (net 52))
 (segment (start 6.35 20.49) (end 6.52 20.49) (width 0.25) (layer B.Cu) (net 52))
 (segment (start 2.54 46.99) (end 7.62 46.99) (width 0.25) (layer B.Cu) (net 48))
 (segment (start 7.62 46.99) (end 12.7 46.99) (width 0.25) (layer B.Cu) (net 48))
 (segment (start 2.54 44.45) (end 7.62 44.45) (width 0.25) (layer B.Cu) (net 49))
 (segment (start 7.62 44.45) (end 12.7 44.45) (width 0.25) (layer B.Cu) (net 49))
 (segment (start 2.54 41.91) (end 7.62 41.91) (width 0.25) (layer B.Cu) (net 50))
 (segment (start 7.62 41.91) (end 12.7 41.91) (width 0.25) (layer B.Cu) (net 50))
 (segment (start 2.54 39.37) (end 7.62 39.37) (width 0.25) (layer B.Cu) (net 51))
 (segment (start 7.62 39.37) (end 12.7 39.37) (width 0.25) (layer B.Cu) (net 51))
 (segment (start 55.88 40.64) (end 55.88 39.54) (width 0.25) (layer B.Cu) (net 27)))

